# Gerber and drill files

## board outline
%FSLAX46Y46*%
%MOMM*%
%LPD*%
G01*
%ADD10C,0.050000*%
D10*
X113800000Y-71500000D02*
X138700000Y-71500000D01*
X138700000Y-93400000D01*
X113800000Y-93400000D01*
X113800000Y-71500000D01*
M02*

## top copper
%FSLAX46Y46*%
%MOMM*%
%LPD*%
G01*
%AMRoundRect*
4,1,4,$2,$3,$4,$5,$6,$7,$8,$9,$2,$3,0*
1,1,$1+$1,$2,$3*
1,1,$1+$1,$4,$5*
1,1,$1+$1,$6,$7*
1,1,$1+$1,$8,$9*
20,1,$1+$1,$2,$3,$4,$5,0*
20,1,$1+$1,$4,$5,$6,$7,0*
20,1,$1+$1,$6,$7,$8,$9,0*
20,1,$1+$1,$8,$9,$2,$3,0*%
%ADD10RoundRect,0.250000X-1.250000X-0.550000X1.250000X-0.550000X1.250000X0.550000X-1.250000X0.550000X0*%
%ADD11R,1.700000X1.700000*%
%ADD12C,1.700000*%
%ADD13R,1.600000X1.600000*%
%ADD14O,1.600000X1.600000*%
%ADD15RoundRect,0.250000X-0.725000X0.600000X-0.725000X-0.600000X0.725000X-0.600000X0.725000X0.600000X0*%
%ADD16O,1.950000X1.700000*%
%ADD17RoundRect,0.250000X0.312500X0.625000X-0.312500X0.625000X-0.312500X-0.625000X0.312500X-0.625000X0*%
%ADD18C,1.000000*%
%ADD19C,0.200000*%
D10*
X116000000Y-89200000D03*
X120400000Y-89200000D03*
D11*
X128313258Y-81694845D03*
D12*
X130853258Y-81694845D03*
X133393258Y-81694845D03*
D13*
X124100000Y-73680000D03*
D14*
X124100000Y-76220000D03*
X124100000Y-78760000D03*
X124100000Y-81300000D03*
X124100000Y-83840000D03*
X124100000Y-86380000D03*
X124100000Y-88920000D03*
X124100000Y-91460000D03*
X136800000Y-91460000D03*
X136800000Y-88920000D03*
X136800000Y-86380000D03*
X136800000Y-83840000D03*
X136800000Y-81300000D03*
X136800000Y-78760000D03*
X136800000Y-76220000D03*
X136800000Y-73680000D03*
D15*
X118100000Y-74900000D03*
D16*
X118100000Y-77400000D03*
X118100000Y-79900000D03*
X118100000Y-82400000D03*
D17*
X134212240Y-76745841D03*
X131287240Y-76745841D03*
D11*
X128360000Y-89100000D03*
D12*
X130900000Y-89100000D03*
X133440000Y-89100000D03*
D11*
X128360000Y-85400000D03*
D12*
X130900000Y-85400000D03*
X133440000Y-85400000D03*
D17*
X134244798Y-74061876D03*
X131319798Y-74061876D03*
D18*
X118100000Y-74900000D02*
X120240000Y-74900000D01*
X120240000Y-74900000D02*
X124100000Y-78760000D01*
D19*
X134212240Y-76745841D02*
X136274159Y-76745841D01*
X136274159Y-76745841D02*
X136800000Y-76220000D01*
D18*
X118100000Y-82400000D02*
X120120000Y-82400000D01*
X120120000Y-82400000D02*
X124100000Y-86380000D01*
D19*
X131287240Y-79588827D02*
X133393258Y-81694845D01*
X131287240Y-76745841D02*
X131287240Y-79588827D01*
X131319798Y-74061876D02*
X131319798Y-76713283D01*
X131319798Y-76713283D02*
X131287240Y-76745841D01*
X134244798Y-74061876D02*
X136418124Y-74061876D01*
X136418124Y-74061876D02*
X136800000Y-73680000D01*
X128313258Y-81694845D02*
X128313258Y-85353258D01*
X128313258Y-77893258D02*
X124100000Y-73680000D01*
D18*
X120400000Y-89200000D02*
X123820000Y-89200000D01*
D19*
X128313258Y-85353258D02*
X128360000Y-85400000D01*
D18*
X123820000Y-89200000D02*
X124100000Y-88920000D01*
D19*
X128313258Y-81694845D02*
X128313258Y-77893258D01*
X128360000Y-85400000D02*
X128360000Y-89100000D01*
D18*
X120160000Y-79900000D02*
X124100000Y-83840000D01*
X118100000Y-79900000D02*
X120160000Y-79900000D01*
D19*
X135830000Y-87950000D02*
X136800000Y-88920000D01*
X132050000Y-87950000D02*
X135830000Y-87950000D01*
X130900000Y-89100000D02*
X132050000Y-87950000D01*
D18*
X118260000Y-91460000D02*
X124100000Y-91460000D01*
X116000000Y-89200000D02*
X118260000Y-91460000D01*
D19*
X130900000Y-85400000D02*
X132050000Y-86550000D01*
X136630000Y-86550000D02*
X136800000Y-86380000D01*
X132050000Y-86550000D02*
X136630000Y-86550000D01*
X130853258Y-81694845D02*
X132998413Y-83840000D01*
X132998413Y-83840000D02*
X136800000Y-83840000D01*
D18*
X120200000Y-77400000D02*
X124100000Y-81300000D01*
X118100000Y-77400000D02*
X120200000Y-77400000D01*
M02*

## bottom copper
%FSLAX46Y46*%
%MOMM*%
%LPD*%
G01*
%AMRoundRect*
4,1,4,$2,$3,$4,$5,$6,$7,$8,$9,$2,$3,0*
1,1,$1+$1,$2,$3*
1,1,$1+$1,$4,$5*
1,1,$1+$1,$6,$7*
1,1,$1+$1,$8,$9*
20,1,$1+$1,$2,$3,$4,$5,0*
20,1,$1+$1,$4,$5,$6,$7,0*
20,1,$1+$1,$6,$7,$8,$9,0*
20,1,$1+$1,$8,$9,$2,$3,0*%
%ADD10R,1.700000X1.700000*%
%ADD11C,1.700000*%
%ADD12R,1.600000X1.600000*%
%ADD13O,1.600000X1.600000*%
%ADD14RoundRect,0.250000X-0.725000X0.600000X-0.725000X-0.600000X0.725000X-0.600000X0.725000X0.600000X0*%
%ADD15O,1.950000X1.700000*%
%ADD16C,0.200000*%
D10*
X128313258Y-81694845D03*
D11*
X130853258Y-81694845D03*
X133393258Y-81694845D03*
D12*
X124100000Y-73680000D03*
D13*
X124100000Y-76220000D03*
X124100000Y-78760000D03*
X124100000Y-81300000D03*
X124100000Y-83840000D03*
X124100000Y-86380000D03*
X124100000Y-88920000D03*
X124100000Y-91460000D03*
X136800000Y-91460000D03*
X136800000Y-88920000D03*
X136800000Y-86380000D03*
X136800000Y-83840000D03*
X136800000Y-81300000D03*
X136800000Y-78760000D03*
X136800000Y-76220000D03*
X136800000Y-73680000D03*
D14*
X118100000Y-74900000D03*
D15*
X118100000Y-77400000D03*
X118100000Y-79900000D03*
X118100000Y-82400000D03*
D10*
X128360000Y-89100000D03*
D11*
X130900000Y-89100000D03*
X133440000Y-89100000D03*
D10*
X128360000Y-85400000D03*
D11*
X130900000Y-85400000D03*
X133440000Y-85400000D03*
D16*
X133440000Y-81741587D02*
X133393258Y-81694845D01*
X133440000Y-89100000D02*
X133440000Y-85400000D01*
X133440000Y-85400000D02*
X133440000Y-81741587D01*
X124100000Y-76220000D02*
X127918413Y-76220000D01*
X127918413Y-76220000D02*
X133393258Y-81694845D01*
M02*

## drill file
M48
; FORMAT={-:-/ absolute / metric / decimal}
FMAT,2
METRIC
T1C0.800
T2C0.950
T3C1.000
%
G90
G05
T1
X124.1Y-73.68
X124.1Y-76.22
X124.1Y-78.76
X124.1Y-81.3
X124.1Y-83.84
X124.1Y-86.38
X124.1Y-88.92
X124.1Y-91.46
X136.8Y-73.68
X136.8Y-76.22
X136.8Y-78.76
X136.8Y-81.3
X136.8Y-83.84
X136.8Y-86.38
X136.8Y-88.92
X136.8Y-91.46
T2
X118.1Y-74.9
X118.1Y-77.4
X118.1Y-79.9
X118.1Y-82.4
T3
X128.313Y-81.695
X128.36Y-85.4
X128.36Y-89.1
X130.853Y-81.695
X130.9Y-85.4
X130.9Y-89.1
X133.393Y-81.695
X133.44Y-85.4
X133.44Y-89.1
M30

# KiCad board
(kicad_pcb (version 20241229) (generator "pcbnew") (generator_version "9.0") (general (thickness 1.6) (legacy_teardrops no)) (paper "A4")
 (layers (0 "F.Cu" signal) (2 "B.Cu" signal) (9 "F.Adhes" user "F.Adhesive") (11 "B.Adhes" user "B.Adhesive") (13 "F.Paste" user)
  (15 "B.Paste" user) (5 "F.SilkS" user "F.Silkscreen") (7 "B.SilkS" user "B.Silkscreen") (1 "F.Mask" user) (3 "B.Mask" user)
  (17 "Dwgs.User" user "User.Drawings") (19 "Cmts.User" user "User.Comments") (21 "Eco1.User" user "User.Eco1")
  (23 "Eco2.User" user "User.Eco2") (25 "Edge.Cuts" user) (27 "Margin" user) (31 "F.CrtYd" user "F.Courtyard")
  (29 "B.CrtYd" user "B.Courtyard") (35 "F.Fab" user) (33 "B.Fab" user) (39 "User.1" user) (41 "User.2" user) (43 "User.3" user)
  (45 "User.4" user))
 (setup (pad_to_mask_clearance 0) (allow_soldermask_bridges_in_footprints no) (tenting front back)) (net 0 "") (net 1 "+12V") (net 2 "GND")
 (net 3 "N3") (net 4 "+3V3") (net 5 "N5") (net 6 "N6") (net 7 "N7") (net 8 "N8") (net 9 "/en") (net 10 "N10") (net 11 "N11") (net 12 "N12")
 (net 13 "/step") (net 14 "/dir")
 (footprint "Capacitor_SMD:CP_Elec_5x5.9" (layer "F.Cu") (at 118.2 89.2)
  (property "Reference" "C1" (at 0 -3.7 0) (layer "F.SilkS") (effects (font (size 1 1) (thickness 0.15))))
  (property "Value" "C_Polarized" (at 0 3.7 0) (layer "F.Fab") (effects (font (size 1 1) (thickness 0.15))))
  (pad "1" smd roundrect (at -2.2 0) (size 3 1.6) (layers "F.Cu" "F.Mask" "F.Paste") (roundrect_rratio 0.15625) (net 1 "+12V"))
  (pad "2" smd roundrect (at 2.2 0) (size 3 1.6) (layers "F.Cu" "F.Mask" "F.Paste") (roundrect_rratio 0.15625) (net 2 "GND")))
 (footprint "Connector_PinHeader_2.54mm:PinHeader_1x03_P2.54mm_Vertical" (layer "F.Cu") (at 128.313258 81.694845 90)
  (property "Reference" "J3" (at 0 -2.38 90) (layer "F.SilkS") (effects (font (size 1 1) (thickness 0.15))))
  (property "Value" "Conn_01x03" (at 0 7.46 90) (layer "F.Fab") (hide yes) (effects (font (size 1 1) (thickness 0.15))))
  (pad "1" thru_hole rect (at 0 0 90) (size 1.7 1.7) (drill 1) (layers "*.Cu" "*.Mask") (remove_unused_layers no) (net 2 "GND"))
  (pad "2" thru_hole circle (at 0 2.54 90) (size 1.7 1.7) (drill 1) (layers "*.Cu" "*.Mask") (remove_unused_layers no) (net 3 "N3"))
  (pad "3" thru_hole circle (at 0 5.08 90) (size 1.7 1.7) (drill 1) (layers "*.Cu" "*.Mask") (remove_unused_layers no) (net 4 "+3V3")))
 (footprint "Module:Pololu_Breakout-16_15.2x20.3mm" (layer "F.Cu") (at 124.1 73.68)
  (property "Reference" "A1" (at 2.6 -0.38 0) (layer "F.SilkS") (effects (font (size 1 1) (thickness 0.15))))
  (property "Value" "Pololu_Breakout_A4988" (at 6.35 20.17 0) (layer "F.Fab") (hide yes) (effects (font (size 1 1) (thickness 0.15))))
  (pad "1" thru_hole rect (at 0 0) (size 1.6 1.6) (drill 0.8) (layers "*.Cu" "*.Mask") (remove_unused_layers no) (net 2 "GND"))
  (pad "2" thru_hole oval (at 0 2.54) (size 1.6 1.6) (drill 0.8) (layers "*.Cu" "*.Mask") (remove_unused_layers no) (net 4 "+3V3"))
  (pad "3" thru_hole oval (at 0 5.08) (size 1.6 1.6) (drill 0.8) (layers "*.Cu" "*.Mask") (remove_unused_layers no) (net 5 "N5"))
  (pad "4" thru_hole oval (at 0 7.62) (size 1.6 1.6) (drill 0.8) (layers "*.Cu" "*.Mask") (remove_unused_layers no) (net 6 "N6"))
  (pad "5" thru_hole oval (at 0 10.16) (size 1.6 1.6) (drill 0.8) (layers "*.Cu" "*.Mask") (remove_unused_layers no) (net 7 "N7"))
  (pad "6" thru_hole oval (at 0 12.7) (size 1.6 1.6) (drill 0.8) (layers "*.Cu" "*.Mask") (remove_unused_layers no) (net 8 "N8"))
  (pad "7" thru_hole oval (at 0 15.24) (size 1.6 1.6) (drill 0.8) (layers "*.Cu" "*.Mask") (remove_unused_layers no) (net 2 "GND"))
  (pad "8" thru_hole oval (at 0 17.78) (size 1.6 1.6) (drill 0.8) (layers "*.Cu" "*.Mask") (remove_unused_layers no) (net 1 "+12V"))
  (pad "9" thru_hole oval (at 12.7 17.78) (size 1.6 1.6) (drill 0.8) (layers "*.Cu" "*.Mask") (remove_unused_layers no) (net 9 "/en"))
  (pad "10" thru_hole oval (at 12.7 15.24) (size 1.6 1.6) (drill 0.8) (layers "*.Cu" "*.Mask") (remove_unused_layers no) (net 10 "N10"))
  (pad "11" thru_hole oval (at 12.7 12.7) (size 1.6 1.6) (drill 0.8) (layers "*.Cu" "*.Mask") (remove_unused_layers no) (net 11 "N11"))
  (pad "12" thru_hole oval (at 12.7 10.16) (size 1.6 1.6) (drill 0.8) (layers "*.Cu" "*.Mask") (remove_unused_layers no) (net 3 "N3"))
  (pad "13" thru_hole oval (at 12.7 7.62) (size 1.6 1.6) (drill 0.8) (layers "*.Cu" "*.Mask") (remove_unused_layers no) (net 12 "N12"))
  (pad "14" thru_hole oval (at 12.7 5.08) (size 1.6 1.6) (drill 0.8) (layers "*.Cu" "*.Mask") (remove_unused_layers no) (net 12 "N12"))
  (pad "15" thru_hole oval (at 12.7 2.54) (size 1.6 1.6) (drill 0.8) (layers "*.Cu" "*.Mask") (remove_unused_layers no) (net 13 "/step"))
  (pad "16" thru_hole oval (at 12.7 0) (size 1.6 1.6) (drill 0.8) (layers "*.Cu" "*.Mask") (remove_unused_layers no) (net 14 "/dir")))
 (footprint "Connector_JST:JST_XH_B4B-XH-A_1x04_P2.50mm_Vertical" (layer "F.Cu") (at 118.1 74.9 -90)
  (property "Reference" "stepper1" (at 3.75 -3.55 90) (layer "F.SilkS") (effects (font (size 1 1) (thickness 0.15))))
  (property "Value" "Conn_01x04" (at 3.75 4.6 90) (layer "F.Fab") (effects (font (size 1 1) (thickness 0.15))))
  (pad "1" thru_hole roundrect (at 0 0 270) (size 1.7 1.95) (drill 0.95) (layers "*.Cu" "*.Mask") (remove_unused_layers no)
   (roundrect_rratio 0.147059) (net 5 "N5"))
  (pad "2" thru_hole oval (at 2.5 0 270) (size 1.7 1.95) (drill 0.95) (layers "*.Cu" "*.Mask") (remove_unused_layers no) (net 6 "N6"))
  (pad "3" thru_hole oval (at 5 0 270) (size 1.7 1.95) (drill 0.95) (layers "*.Cu" "*.Mask") (remove_unused_layers no) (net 7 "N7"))
  (pad "4" thru_hole oval (at 7.5 0 270) (size 1.7 1.95) (drill 0.95) (layers "*.Cu" "*.Mask") (remove_unused_layers no) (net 8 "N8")))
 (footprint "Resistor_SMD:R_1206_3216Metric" (layer "F.Cu") (at 132.74974 76.745841 180)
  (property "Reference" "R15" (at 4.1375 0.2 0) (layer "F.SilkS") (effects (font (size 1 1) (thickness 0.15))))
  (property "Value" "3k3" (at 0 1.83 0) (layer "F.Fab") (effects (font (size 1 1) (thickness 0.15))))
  (pad "1" smd roundrect (at -1.4625 0 180) (size 1.125 1.75) (layers "F.Cu" "F.Mask" "F.Paste") (roundrect_rratio 0.222222)
   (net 13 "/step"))
  (pad "2" smd roundrect (at 1.4625 0 180) (size 1.125 1.75) (layers "F.Cu" "F.Mask" "F.Paste") (roundrect_rratio 0.222222) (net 4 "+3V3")))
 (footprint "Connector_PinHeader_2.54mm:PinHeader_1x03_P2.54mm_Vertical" (layer "F.Cu") (at 128.36 89.1 90)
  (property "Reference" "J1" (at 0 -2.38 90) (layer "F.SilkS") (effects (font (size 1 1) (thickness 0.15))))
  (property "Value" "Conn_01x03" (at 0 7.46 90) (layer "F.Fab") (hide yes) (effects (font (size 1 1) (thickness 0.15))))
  (pad "1" thru_hole rect (at 0 0 90) (size 1.7 1.7) (drill 1) (layers "*.Cu" "*.Mask") (remove_unused_layers no) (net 2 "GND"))
  (pad "2" thru_hole circle (at 0 2.54 90) (size 1.7 1.7) (drill 1) (layers "*.Cu" "*.Mask") (remove_unused_layers no) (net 10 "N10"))
  (pad "3" thru_hole circle (at 0 5.08 90) (size 1.7 1.7) (drill 1) (layers "*.Cu" "*.Mask") (remove_unused_layers no) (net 4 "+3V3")))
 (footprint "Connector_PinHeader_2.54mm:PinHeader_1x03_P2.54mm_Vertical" (layer "F.Cu") (at 128.36 85.4 90)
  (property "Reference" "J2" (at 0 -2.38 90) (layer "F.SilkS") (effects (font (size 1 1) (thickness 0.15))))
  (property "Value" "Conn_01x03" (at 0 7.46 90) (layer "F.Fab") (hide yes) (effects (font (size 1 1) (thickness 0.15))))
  (pad "1" thru_hole rect (at 0 0 90) (size 1.7 1.7) (drill 1) (layers "*.Cu" "*.Mask") (remove_unused_layers no) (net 2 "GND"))
  (pad "2" thru_hole circle (at 0 2.54 90) (size 1.7 1.7) (drill 1) (layers "*.Cu" "*.Mask") (remove_unused_layers no) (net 11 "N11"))
  (pad "3" thru_hole circle (at 0 5.08 90) (size 1.7 1.7) (drill 1) (layers "*.Cu" "*.Mask") (remove_unused_layers no) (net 4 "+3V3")))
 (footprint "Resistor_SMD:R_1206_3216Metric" (layer "F.Cu") (at 132.782298 74.061876 180)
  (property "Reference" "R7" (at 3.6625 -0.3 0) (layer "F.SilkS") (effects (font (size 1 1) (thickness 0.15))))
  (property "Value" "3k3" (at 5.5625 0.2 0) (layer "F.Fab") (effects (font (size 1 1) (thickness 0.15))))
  (pad "1" smd roundrect (at -1.4625 0 180) (size 1.125 1.75) (layers "F.Cu" "F.Mask" "F.Paste") (roundrect_rratio 0.222222) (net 14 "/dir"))
  (pad "2" smd roundrect (at 1.4625 0 180) (size 1.125 1.75) (layers "F.Cu" "F.Mask" "F.Paste") (roundrect_rratio 0.222222) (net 4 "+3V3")))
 (gr_rect (start 113.8 71.5) (end 138.7 93.4) (stroke (width 0.05) (type default)) (fill no) (layer "Edge.Cuts"))
 (segment (start 118.1 74.9) (end 120.24 74.9) (width 1) (layer "F.Cu") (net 5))
 (segment (start 120.24 74.9) (end 124.1 78.76) (width 1) (layer "F.Cu") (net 5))
 (segment (start 134.21224 76.745841) (end 136.274159 76.745841) (width 0.2) (layer "F.Cu") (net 13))
 (segment (start 136.274159 76.745841) (end 136.8 76.22) (width 0.2) (layer "F.Cu") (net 13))
 (segment (start 118.1 82.4) (end 120.12 82.4) (width 1) (layer "F.Cu") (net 8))
 (segment (start 120.12 82.4) (end 124.1 86.38) (width 1) (layer "F.Cu") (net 8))
 (segment (start 131.28724 79.588827) (end 133.393258 81.694845) (width 0.2) (layer "F.Cu") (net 4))
 (segment (start 131.28724 76.745841) (end 131.28724 79.588827) (width 0.2) (layer "F.Cu") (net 4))
 (segment (start 131.319798 74.061876) (end 131.319798 76.713283) (width 0.2) (layer "F.Cu") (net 4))
 (segment (start 131.319798 76.713283) (end 131.28724 76.745841) (width 0.2) (layer "F.Cu") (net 4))
 (segment (start 133.44 81.741587) (end 133.393258 81.694845) (width 0.2) (layer "B.Cu") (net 4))
 (segment (start 133.44 89.1) (end 133.44 85.4) (width 0.2) (layer "B.Cu") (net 4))
 (segment (start 133.44 85.4) (end 133.44 81.741587) (width 0.2) (layer "B.Cu") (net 4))
 (segment (start 124.1 76.22) (end 127.918413 76.22) (width 0.2) (layer "B.Cu") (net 4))
 (segment (start 127.918413 76.22) (end 133.393258 81.694845) (width 0.2) (layer "B.Cu") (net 4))
 (segment (start 134.244798 74.061876) (end 136.418124 74.061876) (width 0.2) (layer "F.Cu") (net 14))
 (segment (start 136.418124 74.061876) (end 136.8 73.68) (width 0.2) (layer "F.Cu") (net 14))
 (segment (start 128.313258 81.694845) (end 128.313258 85.353258) (width 0.2) (layer "F.Cu") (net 2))
 (segment (start 128.313258 77.893258) (end 124.1 73.68) (width 0.2) (layer "F.Cu") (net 2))
 (segment (start 120.4 89.2) (end 123.82 89.2) (width 1) (layer "F.Cu") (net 2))
 (segment (start 128.313258 85.353258) (end 128.36 85.4) (width 0.2) (layer "F.Cu") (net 2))
 (segment (start 123.82 89.2) (end 124.1 88.92) (width 1) (layer "F.Cu") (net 2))
 (segment (start 128.313258 81.694845) (end 128.313258 77.893258) (width 0.2) (layer "F.Cu") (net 2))
 (segment (start 128.36 85.4) (end 128.36 89.1) (width 0.2) (layer "F.Cu") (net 2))
 (segment (start 120.16 79.9) (end 124.1 83.84) (width 1) (layer "F.Cu") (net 7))
 (segment (start 118.1 79.9) (end 120.16 79.9) (width 1) (layer "F.Cu") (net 7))
 (segment (start 135.83 87.95) (end 136.8 88.92) (width 0.2) (layer "F.Cu") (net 10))
 (segment (start 132.05 87.95) (end 135.83 87.95) (width 0.2) (layer "F.Cu") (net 10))
 (segment (start 130.9 89.1) (end 132.05 87.95) (width 0.2) (layer "F.Cu") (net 10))
 (segment (start 118.26 91.46) (end 124.1 91.46) (width 1) (layer "F.Cu") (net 1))
 (segment (start 116 89.2) (end 118.26 91.46) (width 1) (layer "F.Cu") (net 1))
 (segment (start 130.9 85.4) (end 132.05 86.55) (width 0.2) (layer "F.Cu") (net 11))
 (segment (start 136.63 86.55) (end 136.8 86.38) (width 0.2) (layer "F.Cu") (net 11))
 (segment (start 132.05 86.55) (end 136.63 86.55) (width 0.2) (layer "F.Cu") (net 11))
 (segment (start 130.853258 81.694845) (end 132.998413 83.84) (width 0.2) (layer "F.Cu") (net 3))
 (segment (start 132.998413 83.84) (end 136.8 83.84) (width 0.2) (layer "F.Cu") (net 3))
 (segment (start 120.2 77.4) (end 124.1 81.3) (width 1) (layer "F.Cu") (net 6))
 (segment (start 118.1 77.4) (end 120.2 77.4) (width 1) (layer "F.Cu") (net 6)))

